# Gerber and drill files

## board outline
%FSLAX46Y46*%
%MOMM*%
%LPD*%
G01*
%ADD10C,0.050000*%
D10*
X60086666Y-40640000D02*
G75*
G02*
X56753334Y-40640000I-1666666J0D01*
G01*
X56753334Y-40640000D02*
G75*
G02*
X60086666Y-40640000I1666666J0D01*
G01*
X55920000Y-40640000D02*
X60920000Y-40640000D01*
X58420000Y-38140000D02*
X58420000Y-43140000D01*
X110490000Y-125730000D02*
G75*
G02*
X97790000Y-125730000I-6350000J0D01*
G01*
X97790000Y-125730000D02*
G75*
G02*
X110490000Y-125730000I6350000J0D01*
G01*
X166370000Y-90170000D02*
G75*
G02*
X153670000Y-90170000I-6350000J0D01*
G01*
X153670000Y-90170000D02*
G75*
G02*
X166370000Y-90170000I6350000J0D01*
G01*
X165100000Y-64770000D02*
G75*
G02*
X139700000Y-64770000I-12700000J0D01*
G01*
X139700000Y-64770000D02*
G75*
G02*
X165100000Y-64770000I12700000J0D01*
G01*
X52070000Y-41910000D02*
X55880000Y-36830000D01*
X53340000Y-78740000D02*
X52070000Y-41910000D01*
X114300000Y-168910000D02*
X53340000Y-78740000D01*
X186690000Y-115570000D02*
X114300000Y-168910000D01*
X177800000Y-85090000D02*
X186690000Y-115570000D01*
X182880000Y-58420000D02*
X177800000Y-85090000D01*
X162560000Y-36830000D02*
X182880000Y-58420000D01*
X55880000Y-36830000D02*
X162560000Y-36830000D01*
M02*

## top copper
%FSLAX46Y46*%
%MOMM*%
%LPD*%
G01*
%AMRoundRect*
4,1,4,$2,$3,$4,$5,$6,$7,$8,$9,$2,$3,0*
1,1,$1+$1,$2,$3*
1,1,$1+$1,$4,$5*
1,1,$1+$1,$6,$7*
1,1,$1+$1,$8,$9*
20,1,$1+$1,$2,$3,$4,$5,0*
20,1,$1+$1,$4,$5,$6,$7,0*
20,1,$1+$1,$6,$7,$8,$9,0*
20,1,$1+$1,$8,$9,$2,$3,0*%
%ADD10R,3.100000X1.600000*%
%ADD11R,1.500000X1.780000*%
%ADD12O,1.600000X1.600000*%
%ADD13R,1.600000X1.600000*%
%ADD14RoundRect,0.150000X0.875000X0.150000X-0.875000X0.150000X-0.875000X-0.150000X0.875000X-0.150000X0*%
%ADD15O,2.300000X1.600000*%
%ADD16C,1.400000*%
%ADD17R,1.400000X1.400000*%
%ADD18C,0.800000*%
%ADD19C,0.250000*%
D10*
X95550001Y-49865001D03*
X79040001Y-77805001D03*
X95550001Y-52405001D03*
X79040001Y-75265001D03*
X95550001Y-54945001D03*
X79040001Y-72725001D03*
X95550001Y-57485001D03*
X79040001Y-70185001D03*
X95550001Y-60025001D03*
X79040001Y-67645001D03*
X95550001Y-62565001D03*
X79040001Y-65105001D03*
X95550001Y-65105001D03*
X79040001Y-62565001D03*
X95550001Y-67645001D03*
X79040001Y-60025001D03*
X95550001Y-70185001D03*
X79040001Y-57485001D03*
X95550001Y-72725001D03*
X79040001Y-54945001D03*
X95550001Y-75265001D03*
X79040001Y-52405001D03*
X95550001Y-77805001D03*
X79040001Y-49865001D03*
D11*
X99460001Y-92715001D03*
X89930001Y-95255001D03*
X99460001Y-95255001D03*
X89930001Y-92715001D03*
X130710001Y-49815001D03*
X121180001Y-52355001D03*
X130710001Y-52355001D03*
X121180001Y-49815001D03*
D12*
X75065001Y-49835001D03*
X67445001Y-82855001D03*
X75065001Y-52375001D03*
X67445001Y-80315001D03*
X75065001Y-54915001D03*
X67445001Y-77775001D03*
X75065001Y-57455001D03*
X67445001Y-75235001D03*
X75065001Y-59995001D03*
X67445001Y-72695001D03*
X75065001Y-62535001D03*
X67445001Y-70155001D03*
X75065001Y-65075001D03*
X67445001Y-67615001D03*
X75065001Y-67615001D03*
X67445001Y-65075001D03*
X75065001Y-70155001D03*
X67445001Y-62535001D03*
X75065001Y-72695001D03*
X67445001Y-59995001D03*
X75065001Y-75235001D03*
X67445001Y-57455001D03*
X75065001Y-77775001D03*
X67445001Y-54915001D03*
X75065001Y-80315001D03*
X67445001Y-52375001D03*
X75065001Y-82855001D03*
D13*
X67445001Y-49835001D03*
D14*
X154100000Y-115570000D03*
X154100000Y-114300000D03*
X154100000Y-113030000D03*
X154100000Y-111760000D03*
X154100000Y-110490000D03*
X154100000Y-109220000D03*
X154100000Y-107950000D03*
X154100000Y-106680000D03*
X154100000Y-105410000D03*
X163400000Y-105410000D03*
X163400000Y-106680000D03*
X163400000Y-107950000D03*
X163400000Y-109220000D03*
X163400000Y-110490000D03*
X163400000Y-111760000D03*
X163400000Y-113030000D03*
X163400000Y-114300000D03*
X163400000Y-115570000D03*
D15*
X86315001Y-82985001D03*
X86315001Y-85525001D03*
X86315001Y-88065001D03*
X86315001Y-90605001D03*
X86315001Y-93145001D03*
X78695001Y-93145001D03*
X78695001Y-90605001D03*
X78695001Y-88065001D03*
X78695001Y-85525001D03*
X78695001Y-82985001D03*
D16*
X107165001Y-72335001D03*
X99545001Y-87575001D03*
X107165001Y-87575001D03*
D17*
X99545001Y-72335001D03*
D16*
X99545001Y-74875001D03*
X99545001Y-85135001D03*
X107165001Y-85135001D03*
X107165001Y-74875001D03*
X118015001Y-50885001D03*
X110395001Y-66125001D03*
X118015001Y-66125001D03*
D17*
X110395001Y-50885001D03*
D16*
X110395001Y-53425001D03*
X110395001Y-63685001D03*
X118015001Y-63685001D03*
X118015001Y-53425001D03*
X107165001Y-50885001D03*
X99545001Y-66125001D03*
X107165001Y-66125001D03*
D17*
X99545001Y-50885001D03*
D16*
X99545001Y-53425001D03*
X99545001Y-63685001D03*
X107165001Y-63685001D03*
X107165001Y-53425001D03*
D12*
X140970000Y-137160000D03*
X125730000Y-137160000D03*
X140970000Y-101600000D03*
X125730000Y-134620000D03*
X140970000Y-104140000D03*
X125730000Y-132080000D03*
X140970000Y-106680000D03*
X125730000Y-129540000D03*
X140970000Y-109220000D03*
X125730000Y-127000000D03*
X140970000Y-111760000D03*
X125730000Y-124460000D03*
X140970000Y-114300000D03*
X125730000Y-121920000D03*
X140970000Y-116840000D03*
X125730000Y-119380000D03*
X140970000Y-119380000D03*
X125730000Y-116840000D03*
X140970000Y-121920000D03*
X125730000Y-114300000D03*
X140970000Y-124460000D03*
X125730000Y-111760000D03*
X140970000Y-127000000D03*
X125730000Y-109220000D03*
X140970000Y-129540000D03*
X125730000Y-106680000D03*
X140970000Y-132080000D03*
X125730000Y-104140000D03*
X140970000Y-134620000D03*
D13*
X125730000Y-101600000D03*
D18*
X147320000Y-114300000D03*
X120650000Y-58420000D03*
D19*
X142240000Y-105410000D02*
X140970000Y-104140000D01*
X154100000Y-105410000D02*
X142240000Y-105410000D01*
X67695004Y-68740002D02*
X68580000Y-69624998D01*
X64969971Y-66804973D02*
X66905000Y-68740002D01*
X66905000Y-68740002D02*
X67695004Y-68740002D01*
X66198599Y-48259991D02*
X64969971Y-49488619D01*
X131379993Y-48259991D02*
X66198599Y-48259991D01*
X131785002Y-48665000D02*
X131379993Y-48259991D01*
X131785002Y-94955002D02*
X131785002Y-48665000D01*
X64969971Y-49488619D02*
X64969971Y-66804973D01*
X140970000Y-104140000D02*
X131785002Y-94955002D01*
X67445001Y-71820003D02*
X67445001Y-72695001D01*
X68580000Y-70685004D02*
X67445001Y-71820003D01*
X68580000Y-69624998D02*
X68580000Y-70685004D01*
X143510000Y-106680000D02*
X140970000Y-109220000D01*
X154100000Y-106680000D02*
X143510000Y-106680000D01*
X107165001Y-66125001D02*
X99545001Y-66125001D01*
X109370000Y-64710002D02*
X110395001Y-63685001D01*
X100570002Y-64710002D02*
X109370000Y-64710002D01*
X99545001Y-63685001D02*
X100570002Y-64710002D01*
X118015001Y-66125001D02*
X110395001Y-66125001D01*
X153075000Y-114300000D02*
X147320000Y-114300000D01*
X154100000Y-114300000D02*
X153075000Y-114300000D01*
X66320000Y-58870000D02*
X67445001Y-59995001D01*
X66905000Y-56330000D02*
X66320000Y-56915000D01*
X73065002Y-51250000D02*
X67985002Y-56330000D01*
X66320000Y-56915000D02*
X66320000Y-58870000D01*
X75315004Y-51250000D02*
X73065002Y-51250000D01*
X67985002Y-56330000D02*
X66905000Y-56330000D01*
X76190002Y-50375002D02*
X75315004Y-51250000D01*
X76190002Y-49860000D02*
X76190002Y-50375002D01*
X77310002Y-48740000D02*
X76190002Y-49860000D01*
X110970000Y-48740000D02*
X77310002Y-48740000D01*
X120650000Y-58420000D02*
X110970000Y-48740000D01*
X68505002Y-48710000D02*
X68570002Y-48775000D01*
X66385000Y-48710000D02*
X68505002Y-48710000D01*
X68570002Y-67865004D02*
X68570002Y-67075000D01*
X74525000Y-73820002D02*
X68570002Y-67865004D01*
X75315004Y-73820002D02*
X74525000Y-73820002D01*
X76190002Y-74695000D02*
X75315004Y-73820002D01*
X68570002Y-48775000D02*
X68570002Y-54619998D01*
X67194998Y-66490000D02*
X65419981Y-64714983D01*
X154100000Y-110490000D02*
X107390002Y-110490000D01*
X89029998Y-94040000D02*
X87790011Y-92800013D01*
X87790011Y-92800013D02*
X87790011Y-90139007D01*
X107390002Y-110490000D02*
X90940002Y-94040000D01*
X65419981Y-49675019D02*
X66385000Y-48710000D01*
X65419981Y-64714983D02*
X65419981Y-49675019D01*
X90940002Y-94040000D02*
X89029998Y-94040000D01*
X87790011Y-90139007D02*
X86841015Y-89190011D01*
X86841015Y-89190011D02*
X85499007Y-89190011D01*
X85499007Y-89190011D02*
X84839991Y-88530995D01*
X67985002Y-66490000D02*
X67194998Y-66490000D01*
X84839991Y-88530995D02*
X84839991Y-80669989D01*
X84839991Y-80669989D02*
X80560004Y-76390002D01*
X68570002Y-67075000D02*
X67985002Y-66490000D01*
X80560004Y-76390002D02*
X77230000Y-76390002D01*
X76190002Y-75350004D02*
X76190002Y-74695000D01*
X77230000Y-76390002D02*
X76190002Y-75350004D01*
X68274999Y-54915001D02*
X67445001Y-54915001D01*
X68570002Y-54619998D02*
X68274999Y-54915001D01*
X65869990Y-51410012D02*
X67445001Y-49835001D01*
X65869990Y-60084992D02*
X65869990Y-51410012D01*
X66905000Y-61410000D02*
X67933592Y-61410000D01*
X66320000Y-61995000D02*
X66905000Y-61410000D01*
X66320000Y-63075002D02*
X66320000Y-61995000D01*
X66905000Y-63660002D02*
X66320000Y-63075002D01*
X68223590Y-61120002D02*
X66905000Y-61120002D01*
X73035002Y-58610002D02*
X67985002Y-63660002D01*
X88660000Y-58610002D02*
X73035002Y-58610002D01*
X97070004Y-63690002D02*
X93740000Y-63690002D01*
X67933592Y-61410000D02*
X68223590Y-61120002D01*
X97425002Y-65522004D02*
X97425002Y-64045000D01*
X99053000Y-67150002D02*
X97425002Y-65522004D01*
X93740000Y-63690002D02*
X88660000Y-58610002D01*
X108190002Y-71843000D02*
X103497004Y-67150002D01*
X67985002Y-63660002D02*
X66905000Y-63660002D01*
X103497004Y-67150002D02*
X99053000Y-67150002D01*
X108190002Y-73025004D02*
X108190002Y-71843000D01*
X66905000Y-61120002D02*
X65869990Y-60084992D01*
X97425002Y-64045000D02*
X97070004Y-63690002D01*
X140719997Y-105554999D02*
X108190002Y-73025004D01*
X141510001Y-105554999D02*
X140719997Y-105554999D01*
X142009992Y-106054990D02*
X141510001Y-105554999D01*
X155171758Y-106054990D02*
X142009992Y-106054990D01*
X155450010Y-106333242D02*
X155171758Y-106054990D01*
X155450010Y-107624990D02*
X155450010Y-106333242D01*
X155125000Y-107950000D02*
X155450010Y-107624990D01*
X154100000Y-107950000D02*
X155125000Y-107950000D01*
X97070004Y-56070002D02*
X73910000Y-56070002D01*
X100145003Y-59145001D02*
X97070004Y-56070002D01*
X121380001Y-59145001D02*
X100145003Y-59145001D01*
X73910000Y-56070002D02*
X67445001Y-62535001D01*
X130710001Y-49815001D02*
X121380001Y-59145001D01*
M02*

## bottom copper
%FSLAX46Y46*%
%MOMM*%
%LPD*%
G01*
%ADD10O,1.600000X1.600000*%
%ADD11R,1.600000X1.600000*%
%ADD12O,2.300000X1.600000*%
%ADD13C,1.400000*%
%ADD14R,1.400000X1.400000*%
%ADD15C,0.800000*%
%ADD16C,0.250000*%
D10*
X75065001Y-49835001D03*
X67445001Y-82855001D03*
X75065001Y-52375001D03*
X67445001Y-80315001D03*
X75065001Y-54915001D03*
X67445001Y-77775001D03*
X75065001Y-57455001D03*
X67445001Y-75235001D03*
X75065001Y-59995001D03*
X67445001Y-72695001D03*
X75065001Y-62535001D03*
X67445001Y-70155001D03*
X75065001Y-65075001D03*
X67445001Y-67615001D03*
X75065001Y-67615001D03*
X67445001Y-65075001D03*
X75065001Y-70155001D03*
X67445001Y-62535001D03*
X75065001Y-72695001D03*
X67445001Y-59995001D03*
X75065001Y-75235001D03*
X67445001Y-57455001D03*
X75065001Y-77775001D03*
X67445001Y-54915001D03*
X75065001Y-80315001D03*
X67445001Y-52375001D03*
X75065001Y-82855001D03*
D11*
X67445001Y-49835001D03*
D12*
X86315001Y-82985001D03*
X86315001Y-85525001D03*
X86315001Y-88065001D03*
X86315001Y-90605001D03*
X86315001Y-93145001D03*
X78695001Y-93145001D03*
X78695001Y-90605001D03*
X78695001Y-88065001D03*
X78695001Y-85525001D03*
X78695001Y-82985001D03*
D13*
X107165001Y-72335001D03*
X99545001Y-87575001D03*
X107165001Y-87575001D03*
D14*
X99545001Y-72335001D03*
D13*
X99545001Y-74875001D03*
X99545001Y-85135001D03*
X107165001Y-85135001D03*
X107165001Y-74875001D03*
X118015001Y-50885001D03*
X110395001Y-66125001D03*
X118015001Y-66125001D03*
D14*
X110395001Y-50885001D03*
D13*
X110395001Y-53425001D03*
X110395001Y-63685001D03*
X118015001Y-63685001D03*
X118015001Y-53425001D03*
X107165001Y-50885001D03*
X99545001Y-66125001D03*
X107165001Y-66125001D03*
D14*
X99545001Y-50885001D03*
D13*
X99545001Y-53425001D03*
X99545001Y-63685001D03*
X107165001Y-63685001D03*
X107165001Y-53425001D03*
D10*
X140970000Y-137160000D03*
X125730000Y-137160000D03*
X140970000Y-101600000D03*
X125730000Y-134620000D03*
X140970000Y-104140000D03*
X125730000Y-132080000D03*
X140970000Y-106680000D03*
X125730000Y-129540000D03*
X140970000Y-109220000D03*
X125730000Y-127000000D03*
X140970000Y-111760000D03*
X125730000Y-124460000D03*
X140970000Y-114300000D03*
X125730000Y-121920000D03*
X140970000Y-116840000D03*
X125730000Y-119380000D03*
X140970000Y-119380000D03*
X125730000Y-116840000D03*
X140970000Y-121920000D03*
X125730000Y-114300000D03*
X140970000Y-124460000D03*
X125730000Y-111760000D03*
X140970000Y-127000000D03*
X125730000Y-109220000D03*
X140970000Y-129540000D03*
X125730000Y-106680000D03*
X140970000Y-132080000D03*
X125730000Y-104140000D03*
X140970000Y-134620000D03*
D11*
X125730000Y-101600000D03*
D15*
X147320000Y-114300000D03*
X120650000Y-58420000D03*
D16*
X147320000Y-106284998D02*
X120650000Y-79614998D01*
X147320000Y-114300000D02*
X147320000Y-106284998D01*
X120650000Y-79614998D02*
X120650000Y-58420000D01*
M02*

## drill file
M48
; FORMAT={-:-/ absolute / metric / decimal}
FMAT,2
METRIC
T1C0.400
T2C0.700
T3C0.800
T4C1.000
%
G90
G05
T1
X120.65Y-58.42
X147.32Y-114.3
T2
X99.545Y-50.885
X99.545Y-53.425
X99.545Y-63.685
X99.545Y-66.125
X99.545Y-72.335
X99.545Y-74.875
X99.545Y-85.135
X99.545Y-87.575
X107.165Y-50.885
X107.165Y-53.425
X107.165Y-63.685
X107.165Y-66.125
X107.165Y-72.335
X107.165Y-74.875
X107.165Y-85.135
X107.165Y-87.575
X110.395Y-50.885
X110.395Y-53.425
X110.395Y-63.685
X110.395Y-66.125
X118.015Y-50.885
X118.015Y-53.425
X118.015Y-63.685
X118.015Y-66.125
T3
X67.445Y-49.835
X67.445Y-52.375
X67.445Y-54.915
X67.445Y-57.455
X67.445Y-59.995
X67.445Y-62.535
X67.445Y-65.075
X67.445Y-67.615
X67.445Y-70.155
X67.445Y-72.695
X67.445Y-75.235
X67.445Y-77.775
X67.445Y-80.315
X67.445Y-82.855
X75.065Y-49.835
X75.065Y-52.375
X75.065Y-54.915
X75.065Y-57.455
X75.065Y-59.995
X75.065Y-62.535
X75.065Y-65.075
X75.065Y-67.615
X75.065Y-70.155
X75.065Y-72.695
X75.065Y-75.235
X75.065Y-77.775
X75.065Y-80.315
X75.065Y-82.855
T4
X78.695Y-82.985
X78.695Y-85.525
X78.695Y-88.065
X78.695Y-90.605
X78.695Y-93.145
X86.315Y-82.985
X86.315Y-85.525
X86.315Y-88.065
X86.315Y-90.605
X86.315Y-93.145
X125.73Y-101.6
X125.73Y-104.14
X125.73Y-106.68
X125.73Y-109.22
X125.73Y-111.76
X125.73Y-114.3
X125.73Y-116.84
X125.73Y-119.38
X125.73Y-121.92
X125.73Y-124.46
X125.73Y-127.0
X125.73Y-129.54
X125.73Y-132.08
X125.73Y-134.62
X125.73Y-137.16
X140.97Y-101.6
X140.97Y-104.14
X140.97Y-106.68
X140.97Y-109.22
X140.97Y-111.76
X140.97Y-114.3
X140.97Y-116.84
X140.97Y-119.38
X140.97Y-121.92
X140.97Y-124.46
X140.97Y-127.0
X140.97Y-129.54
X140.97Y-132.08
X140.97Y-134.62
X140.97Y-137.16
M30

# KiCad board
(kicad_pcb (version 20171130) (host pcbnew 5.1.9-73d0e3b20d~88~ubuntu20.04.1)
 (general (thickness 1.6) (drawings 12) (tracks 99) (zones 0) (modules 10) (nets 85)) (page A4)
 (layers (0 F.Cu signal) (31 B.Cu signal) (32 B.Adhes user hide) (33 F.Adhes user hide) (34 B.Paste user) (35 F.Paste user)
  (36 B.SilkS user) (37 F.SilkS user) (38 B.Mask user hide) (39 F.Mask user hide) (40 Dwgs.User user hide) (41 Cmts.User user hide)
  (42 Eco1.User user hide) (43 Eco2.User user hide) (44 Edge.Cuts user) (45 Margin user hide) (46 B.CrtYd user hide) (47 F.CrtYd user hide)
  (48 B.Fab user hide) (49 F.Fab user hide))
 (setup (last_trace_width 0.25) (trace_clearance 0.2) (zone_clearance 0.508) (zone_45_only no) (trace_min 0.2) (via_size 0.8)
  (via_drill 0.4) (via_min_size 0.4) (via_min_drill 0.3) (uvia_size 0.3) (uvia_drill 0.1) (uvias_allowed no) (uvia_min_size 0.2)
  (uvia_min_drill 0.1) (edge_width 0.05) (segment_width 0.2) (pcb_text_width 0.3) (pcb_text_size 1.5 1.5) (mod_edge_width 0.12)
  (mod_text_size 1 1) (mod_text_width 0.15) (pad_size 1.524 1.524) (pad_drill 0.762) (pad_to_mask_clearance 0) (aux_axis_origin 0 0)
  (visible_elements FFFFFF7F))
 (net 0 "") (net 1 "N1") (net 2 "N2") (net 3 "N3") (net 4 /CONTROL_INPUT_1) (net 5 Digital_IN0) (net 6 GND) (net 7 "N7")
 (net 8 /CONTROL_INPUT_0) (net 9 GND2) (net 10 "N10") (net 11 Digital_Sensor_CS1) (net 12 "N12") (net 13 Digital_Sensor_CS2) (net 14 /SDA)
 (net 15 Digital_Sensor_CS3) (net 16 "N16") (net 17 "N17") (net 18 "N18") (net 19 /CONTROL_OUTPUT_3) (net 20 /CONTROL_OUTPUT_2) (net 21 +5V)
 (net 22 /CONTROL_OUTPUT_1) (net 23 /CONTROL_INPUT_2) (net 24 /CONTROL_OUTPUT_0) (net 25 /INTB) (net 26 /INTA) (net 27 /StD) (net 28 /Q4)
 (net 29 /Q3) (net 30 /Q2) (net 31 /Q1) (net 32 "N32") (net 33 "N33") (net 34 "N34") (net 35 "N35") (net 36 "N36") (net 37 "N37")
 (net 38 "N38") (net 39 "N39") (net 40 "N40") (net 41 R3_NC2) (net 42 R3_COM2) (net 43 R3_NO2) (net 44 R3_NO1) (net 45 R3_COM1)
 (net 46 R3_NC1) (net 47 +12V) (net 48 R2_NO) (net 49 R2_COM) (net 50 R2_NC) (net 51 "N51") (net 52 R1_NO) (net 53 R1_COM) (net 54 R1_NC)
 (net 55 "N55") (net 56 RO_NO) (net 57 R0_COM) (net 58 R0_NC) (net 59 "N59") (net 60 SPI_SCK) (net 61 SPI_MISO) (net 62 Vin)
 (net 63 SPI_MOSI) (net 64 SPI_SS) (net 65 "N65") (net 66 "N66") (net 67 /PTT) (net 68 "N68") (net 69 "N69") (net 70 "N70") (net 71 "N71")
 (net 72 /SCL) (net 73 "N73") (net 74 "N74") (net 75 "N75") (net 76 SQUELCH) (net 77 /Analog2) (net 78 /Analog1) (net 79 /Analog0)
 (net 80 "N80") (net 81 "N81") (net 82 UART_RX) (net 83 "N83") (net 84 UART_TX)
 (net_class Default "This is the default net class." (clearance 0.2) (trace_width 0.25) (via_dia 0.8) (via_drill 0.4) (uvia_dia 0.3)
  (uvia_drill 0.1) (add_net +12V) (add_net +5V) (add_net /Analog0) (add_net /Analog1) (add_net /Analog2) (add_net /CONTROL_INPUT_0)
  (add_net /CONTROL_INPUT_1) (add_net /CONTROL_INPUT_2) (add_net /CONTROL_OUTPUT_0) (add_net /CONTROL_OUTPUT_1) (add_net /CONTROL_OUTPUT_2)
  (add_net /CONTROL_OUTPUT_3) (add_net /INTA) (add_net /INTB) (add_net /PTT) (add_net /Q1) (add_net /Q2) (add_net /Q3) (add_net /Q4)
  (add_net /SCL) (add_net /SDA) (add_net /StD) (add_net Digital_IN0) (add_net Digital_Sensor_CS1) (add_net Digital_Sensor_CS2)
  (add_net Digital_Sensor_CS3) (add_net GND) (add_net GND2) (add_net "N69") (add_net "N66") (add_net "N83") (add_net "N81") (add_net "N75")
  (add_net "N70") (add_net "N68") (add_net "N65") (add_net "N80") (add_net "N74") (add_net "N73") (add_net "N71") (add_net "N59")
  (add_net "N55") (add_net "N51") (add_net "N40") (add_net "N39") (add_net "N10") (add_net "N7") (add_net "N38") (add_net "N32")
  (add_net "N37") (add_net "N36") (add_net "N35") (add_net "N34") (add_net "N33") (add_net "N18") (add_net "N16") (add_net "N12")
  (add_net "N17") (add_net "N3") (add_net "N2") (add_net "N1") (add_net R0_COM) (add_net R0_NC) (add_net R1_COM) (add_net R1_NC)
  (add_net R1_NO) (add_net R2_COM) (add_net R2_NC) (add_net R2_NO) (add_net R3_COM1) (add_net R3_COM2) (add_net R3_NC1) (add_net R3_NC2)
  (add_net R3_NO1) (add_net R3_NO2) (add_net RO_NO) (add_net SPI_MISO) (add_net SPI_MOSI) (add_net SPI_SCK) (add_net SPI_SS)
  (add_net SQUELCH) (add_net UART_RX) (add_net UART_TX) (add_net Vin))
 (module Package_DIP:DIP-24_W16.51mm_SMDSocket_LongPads (layer F.Cu) (at 87.295001 63.835001)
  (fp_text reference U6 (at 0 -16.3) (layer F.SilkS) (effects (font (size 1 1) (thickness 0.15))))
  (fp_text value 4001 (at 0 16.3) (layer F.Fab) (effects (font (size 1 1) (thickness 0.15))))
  (pad 24 smd rect (at 8.255 -13.97) (size 3.1 1.6) (layers F.Cu F.Paste F.Mask))
  (pad 12 smd rect (at -8.255 13.97) (size 3.1 1.6) (layers F.Cu F.Paste F.Mask))
  (pad 23 smd rect (at 8.255 -11.43) (size 3.1 1.6) (layers F.Cu F.Paste F.Mask))
  (pad 11 smd rect (at -8.255 11.43) (size 3.1 1.6) (layers F.Cu F.Paste F.Mask))
  (pad 22 smd rect (at 8.255 -8.89) (size 3.1 1.6) (layers F.Cu F.Paste F.Mask))
  (pad 10 smd rect (at -8.255 8.89) (size 3.1 1.6) (layers F.Cu F.Paste F.Mask))
  (pad 21 smd rect (at 8.255 -6.35) (size 3.1 1.6) (layers F.Cu F.Paste F.Mask))
  (pad 9 smd rect (at -8.255 6.35) (size 3.1 1.6) (layers F.Cu F.Paste F.Mask))
  (pad 20 smd rect (at 8.255 -3.81) (size 3.1 1.6) (layers F.Cu F.Paste F.Mask))
  (pad 8 smd rect (at -8.255 3.81) (size 3.1 1.6) (layers F.Cu F.Paste F.Mask))
  (pad 19 smd rect (at 8.255 -1.27) (size 3.1 1.6) (layers F.Cu F.Paste F.Mask))
  (pad 7 smd rect (at -8.255 1.27) (size 3.1 1.6) (layers F.Cu F.Paste F.Mask))
  (pad 18 smd rect (at 8.255 1.27) (size 3.1 1.6) (layers F.Cu F.Paste F.Mask))
  (pad 6 smd rect (at -8.255 -1.27) (size 3.1 1.6) (layers F.Cu F.Paste F.Mask))
  (pad 17 smd rect (at 8.255 3.81) (size 3.1 1.6) (layers F.Cu F.Paste F.Mask))
  (pad 5 smd rect (at -8.255 -3.81) (size 3.1 1.6) (layers F.Cu F.Paste F.Mask))
  (pad 16 smd rect (at 8.255 6.35) (size 3.1 1.6) (layers F.Cu F.Paste F.Mask))
  (pad 4 smd rect (at -8.255 -6.35) (size 3.1 1.6) (layers F.Cu F.Paste F.Mask))
  (pad 15 smd rect (at 8.255 8.89) (size 3.1 1.6) (layers F.Cu F.Paste F.Mask))
  (pad 3 smd rect (at -8.255 -8.89) (size 3.1 1.6) (layers F.Cu F.Paste F.Mask) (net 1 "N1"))
  (pad 14 smd rect (at 8.255 11.43) (size 3.1 1.6) (layers F.Cu F.Paste F.Mask))
  (pad 2 smd rect (at -8.255 -11.43) (size 3.1 1.6) (layers F.Cu F.Paste F.Mask) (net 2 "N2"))
  (pad 13 smd rect (at 8.255 13.97) (size 3.1 1.6) (layers F.Cu F.Paste F.Mask))
  (pad 1 smd rect (at -8.255 -13.97) (size 3.1 1.6) (layers F.Cu F.Paste F.Mask) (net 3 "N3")))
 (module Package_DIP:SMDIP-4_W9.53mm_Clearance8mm (layer F.Cu) (at 94.695001 93.985001)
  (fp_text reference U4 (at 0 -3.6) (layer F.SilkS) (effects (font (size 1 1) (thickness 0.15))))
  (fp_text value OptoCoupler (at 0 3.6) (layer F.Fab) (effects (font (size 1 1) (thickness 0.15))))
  (pad 4 smd rect (at 4.765 -1.27) (size 1.5 1.78) (layers F.Cu F.Paste F.Mask) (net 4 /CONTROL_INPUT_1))
  (pad 2 smd rect (at -4.765 1.27) (size 1.5 1.78) (layers F.Cu F.Paste F.Mask) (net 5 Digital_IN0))
  (pad 3 smd rect (at 4.765 1.27) (size 1.5 1.78) (layers F.Cu F.Paste F.Mask) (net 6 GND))
  (pad 1 smd rect (at -4.765 -1.27) (size 1.5 1.78) (layers F.Cu F.Paste F.Mask) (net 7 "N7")))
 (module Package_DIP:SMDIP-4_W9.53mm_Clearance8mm (layer F.Cu) (at 125.945001 51.085001)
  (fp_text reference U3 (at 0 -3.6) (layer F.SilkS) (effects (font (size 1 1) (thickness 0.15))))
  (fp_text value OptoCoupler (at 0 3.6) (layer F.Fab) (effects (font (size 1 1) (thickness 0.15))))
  (pad 4 smd rect (at 4.765 -1.27) (size 1.5 1.78) (layers F.Cu F.Paste F.Mask) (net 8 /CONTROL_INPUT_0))
  (pad 2 smd rect (at -4.765 1.27) (size 1.5 1.78) (layers F.Cu F.Paste F.Mask) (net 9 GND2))
  (pad 3 smd rect (at 4.765 1.27) (size 1.5 1.78) (layers F.Cu F.Paste F.Mask) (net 6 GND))
  (pad 1 smd rect (at -4.765 -1.27) (size 1.5 1.78) (layers F.Cu F.Paste F.Mask) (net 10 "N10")))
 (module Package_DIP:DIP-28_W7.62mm (layer F.Cu) (at 67.445001 49.835001)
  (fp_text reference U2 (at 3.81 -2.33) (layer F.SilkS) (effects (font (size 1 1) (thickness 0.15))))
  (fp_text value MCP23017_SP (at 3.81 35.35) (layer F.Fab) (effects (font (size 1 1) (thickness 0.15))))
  (pad 28 thru_hole oval (at 7.62 0) (size 1.6 1.6) (drill 0.8) (layers *.Cu *.Mask) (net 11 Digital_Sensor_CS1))
  (pad 14 thru_hole oval (at 0 33.02) (size 1.6 1.6) (drill 0.8) (layers *.Cu *.Mask) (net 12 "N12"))
  (pad 27 thru_hole oval (at 7.62 2.54) (size 1.6 1.6) (drill 0.8) (layers *.Cu *.Mask) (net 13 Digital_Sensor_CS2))
  (pad 13 thru_hole oval (at 0 30.48) (size 1.6 1.6) (drill 0.8) (layers *.Cu *.Mask) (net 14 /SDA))
  (pad 26 thru_hole oval (at 7.62 5.08) (size 1.6 1.6) (drill 0.8) (layers *.Cu *.Mask) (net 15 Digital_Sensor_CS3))
  (pad 12 thru_hole oval (at 0 27.94) (size 1.6 1.6) (drill 0.8) (layers *.Cu *.Mask) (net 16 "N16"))
  (pad 25 thru_hole oval (at 7.62 7.62) (size 1.6 1.6) (drill 0.8) (layers *.Cu *.Mask) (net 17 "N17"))
  (pad 11 thru_hole oval (at 0 25.4) (size 1.6 1.6) (drill 0.8) (layers *.Cu *.Mask) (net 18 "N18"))
  (pad 24 thru_hole oval (at 7.62 10.16) (size 1.6 1.6) (drill 0.8) (layers *.Cu *.Mask) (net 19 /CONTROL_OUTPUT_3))
  (pad 10 thru_hole oval (at 0 22.86) (size 1.6 1.6) (drill 0.8) (layers *.Cu *.Mask) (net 6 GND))
  (pad 23 thru_hole oval (at 7.62 12.7) (size 1.6 1.6) (drill 0.8) (layers *.Cu *.Mask) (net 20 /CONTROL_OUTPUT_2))
  (pad 9 thru_hole oval (at 0 20.32) (size 1.6 1.6) (drill 0.8) (layers *.Cu *.Mask) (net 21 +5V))
  (pad 22 thru_hole oval (at 7.62 15.24) (size 1.6 1.6) (drill 0.8) (layers *.Cu *.Mask) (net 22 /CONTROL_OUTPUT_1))
  (pad 8 thru_hole oval (at 0 17.78) (size 1.6 1.6) (drill 0.8) (layers *.Cu *.Mask) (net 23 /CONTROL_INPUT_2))
  (pad 21 thru_hole oval (at 7.62 17.78) (size 1.6 1.6) (drill 0.8) (layers *.Cu *.Mask) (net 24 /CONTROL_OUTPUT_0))
  (pad 7 thru_hole oval (at 0 15.24) (size 1.6 1.6) (drill 0.8) (layers *.Cu *.Mask) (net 4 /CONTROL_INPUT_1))
  (pad 20 thru_hole oval (at 7.62 20.32) (size 1.6 1.6) (drill 0.8) (layers *.Cu *.Mask) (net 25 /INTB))
  (pad 6 thru_hole oval (at 0 12.7) (size 1.6 1.6) (drill 0.8) (layers *.Cu *.Mask) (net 8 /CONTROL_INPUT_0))
  (pad 19 thru_hole oval (at 7.62 22.86) (size 1.6 1.6) (drill 0.8) (layers *.Cu *.Mask) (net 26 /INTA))
  (pad 5 thru_hole oval (at 0 10.16) (size 1.6 1.6) (drill 0.8) (layers *.Cu *.Mask) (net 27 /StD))
  (pad 18 thru_hole oval (at 7.62 25.4) (size 1.6 1.6) (drill 0.8) (layers *.Cu *.Mask) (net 21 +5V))
  (pad 4 thru_hole oval (at 0 7.62) (size 1.6 1.6) (drill 0.8) (layers *.Cu *.Mask) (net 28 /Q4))
  (pad 17 thru_hole oval (at 7.62 27.94) (size 1.6 1.6) (drill 0.8) (layers *.Cu *.Mask) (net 6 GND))
  (pad 3 thru_hole oval (at 0 5.08) (size 1.6 1.6) (drill 0.8) (layers *.Cu *.Mask) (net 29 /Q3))
  (pad 16 thru_hole oval (at 7.62 30.48) (size 1.6 1.6) (drill 0.8) (layers *.Cu *.Mask) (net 6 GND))
  (pad 2 thru_hole oval (at 0 2.54) (size 1.6 1.6) (drill 0.8) (layers *.Cu *.Mask) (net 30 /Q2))
  (pad 15 thru_hole oval (at 7.62 33.02) (size 1.6 1.6) (drill 0.8) (layers *.Cu *.Mask) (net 6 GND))
  (pad 1 thru_hole rect (at 0 0) (size 1.6 1.6) (drill 0.8) (layers *.Cu *.Mask) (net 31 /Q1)))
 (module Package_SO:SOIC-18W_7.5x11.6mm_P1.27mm (layer F.Cu) (at 158.75 110.49 180)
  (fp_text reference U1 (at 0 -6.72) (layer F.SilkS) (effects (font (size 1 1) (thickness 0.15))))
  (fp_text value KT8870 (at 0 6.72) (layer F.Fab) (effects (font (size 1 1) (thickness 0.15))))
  (pad 18 smd roundrect (at 4.65 -5.08 180) (size 2.05 0.6) (layers F.Cu F.Paste F.Mask) (roundrect_rratio 0.25) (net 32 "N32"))
  (pad 17 smd roundrect (at 4.65 -3.81 180) (size 2.05 0.6) (layers F.Cu F.Paste F.Mask) (roundrect_rratio 0.25) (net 27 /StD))
  (pad 16 smd roundrect (at 4.65 -2.54 180) (size 2.05 0.6) (layers F.Cu F.Paste F.Mask) (roundrect_rratio 0.25))
  (pad 15 smd roundrect (at 4.65 -1.27 180) (size 2.05 0.6) (layers F.Cu F.Paste F.Mask) (roundrect_rratio 0.25) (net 28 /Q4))
  (pad 14 smd roundrect (at 4.65 0 180) (size 2.05 0.6) (layers F.Cu F.Paste F.Mask) (roundrect_rratio 0.25) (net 29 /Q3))
  (pad 13 smd roundrect (at 4.65 1.27 180) (size 2.05 0.6) (layers F.Cu F.Paste F.Mask) (roundrect_rratio 0.25) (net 30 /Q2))
  (pad 12 smd roundrect (at 4.65 2.54 180) (size 2.05 0.6) (layers F.Cu F.Paste F.Mask) (roundrect_rratio 0.25) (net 31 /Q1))
  (pad 11 smd roundrect (at 4.65 3.81 180) (size 2.05 0.6) (layers F.Cu F.Paste F.Mask) (roundrect_rratio 0.25) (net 21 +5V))
  (pad 10 smd roundrect (at 4.65 5.08 180) (size 2.05 0.6) (layers F.Cu F.Paste F.Mask) (roundrect_rratio 0.25) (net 6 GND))
  (pad 9 smd roundrect (at -4.65 5.08 180) (size 2.05 0.6) (layers F.Cu F.Paste F.Mask) (roundrect_rratio 0.25) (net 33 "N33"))
  (pad 8 smd roundrect (at -4.65 3.81 180) (size 2.05 0.6) (layers F.Cu F.Paste F.Mask) (roundrect_rratio 0.25) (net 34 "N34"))
  (pad 7 smd roundrect (at -4.65 2.54 180) (size 2.05 0.6) (layers F.Cu F.Paste F.Mask) (roundrect_rratio 0.25))
  (pad 6 smd roundrect (at -4.65 1.27 180) (size 2.05 0.6) (layers F.Cu F.Paste F.Mask) (roundrect_rratio 0.25) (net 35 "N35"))
  (pad 5 smd roundrect (at -4.65 0 180) (size 2.05 0.6) (layers F.Cu F.Paste F.Mask) (roundrect_rratio 0.25) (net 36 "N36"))
  (pad 4 smd roundrect (at -4.65 -1.27 180) (size 2.05 0.6) (layers F.Cu F.Paste F.Mask) (roundrect_rratio 0.25) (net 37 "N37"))
  (pad 3 smd roundrect (at -4.65 -2.54 180) (size 2.05 0.6) (layers F.Cu F.Paste F.Mask) (roundrect_rratio 0.25) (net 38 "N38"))
  (pad 2 smd roundrect (at -4.65 -3.81 180) (size 2.05 0.6) (layers F.Cu F.Paste F.Mask) (roundrect_rratio 0.25) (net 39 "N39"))
  (pad 1 smd roundrect (at -4.65 -5.08 180) (size 2.05 0.6) (layers F.Cu F.Paste F.Mask) (roundrect_rratio 0.25) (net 37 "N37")))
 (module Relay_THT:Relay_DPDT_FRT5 (layer F.Cu) (at 78.695001 82.985001)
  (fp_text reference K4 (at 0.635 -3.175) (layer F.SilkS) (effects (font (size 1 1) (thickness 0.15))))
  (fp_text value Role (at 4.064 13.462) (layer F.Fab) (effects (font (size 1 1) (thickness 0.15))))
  (pad 10 thru_hole oval (at 7.62 0) (size 2.3 1.6) (drill 1) (layers *.Cu *.Mask) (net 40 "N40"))
  (pad 9 thru_hole oval (at 7.62 2.54) (size 2.3 1.6) (drill 1) (layers *.Cu *.Mask) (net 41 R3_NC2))
  (pad 8 thru_hole oval (at 7.62 5.08) (size 2.3 1.6) (drill 1) (layers *.Cu *.Mask) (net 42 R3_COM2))
  (pad 7 thru_hole oval (at 7.62 7.62) (size 2.3 1.6) (drill 1) (layers *.Cu *.Mask) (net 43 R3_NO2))
  (pad 6 thru_hole oval (at 7.62 10.16) (size 2.3 1.6) (drill 1) (layers *.Cu *.Mask))
  (pad 5 thru_hole oval (at 0 10.16) (size 2.3 1.6) (drill 1) (layers *.Cu *.Mask))
  (pad 4 thru_hole oval (at 0 7.62) (size 2.3 1.6) (drill 1) (layers *.Cu *.Mask) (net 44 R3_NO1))
  (pad 3 thru_hole oval (at 0 5.08) (size 2.3 1.6) (drill 1) (layers *.Cu *.Mask) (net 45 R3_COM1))
  (pad 2 thru_hole oval (at 0 2.54) (size 2.3 1.6) (drill 1) (layers *.Cu *.Mask) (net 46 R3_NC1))
  (pad 1 thru_hole oval (at 0 0) (size 2.3 1.6) (drill 1) (layers *.Cu *.Mask) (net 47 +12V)))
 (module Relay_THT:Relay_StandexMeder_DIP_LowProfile (layer F.Cu) (at 99.545001 72.335001)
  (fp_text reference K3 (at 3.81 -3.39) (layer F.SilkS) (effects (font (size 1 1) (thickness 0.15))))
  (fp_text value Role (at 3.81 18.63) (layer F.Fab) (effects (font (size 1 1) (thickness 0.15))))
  (pad 14 thru_hole circle (at 7.62 0) (size 1.4 1.4) (drill 0.7) (layers *.Cu *.Mask) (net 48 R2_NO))
  (pad 7 thru_hole circle (at 0 15.24) (size 1.4 1.4) (drill 0.7) (layers *.Cu *.Mask) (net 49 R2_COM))
  (pad 8 thru_hole circle (at 7.62 15.24) (size 1.4 1.4) (drill 0.7) (layers *.Cu *.Mask) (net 49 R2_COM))
  (pad 1 thru_hole rect (at 0 0) (size 1.4 1.4) (drill 0.7) (layers *.Cu *.Mask) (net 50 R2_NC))
  (pad 2 thru_hole circle (at 0 2.54) (size 1.4 1.4) (drill 0.7) (layers *.Cu *.Mask) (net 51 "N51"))
  (pad 6 thru_hole circle (at 0 12.8) (size 1.4 1.4) (drill 0.7) (layers *.Cu *.Mask) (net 47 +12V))
  (pad 9 thru_hole circle (at 7.62 12.8) (size 1.4 1.4) (drill 0.7) (layers *.Cu *.Mask))
  (pad 13 thru_hole circle (at 7.62 2.54) (size 1.4 1.4) (drill 0.7) (layers *.Cu *.Mask)))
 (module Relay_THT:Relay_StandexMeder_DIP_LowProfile (layer F.Cu) (at 110.395001 50.885001)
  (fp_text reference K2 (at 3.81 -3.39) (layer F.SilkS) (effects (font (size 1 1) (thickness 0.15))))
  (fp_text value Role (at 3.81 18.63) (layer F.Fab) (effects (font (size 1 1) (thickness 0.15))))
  (pad 14 thru_hole circle (at 7.62 0) (size 1.4 1.4) (drill 0.7) (layers *.Cu *.Mask) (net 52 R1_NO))
  (pad 7 thru_hole circle (at 0 15.24) (size 1.4 1.4) (drill 0.7) (layers *.Cu *.Mask) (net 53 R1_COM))
  (pad 8 thru_hole circle (at 7.62 15.24) (size 1.4 1.4) (drill 0.7) (layers *.Cu *.Mask) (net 53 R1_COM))
  (pad 1 thru_hole rect (at 0 0) (size 1.4 1.4) (drill 0.7) (layers *.Cu *.Mask) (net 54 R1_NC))
  (pad 2 thru_hole circle (at 0 2.54) (size 1.4 1.4) (drill 0.7) (layers *.Cu *.Mask) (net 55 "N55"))
  (pad 6 thru_hole circle (at 0 12.8) (size 1.4 1.4) (drill 0.7) (layers *.Cu *.Mask) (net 47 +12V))
  (pad 9 thru_hole circle (at 7.62 12.8) (size 1.4 1.4) (drill 0.7) (layers *.Cu *.Mask))
  (pad 13 thru_hole circle (at 7.62 2.54) (size 1.4 1.4) (drill 0.7) (layers *.Cu *.Mask)))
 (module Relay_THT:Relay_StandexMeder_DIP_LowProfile (layer F.Cu) (at 99.545001 50.885001)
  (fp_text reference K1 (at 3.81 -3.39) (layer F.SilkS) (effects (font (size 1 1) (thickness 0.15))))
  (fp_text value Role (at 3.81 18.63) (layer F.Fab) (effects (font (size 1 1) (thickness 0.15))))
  (pad 14 thru_hole circle (at 7.62 0) (size 1.4 1.4) (drill 0.7) (layers *.Cu *.Mask) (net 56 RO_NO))
  (pad 7 thru_hole circle (at 0 15.24) (size 1.4 1.4) (drill 0.7) (layers *.Cu *.Mask) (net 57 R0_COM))
  (pad 8 thru_hole circle (at 7.62 15.24) (size 1.4 1.4) (drill 0.7) (layers *.Cu *.Mask) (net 57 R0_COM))
  (pad 1 thru_hole rect (at 0 0) (size 1.4 1.4) (drill 0.7) (layers *.Cu *.Mask) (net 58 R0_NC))
  (pad 2 thru_hole circle (at 0 2.54) (size 1.4 1.4) (drill 0.7) (layers *.Cu *.Mask) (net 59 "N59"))
  (pad 6 thru_hole circle (at 0 12.8) (size 1.4 1.4) (drill 0.7) (layers *.Cu *.Mask) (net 47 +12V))
  (pad 9 thru_hole circle (at 7.62 12.8) (size 1.4 1.4) (drill 0.7) (layers *.Cu *.Mask))
  (pad 13 thru_hole circle (at 7.62 2.54) (size 1.4 1.4) (drill 0.7) (layers *.Cu *.Mask)))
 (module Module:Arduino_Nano (layer F.Cu) (at 125.73 101.6)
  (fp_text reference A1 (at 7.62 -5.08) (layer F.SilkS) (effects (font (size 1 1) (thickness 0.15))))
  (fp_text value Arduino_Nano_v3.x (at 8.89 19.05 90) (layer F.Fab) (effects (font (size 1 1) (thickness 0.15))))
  (pad 16 thru_hole oval (at 15.24 35.56) (size 1.6 1.6) (drill 1) (layers *.Cu *.Mask) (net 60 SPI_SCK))
  (pad 15 thru_hole oval (at 0 35.56) (size 1.6 1.6) (drill 1) (layers *.Cu *.Mask) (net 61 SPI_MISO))
  (pad 30 thru_hole oval (at 15.24 0) (size 1.6 1.6) (drill 1) (layers *.Cu *.Mask) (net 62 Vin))
  (pad 14 thru_hole oval (at 0 33.02) (size 1.6 1.6) (drill 1) (layers *.Cu *.Mask) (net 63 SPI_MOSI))
  (pad 29 thru_hole oval (at 15.24 2.54) (size 1.6 1.6) (drill 1) (layers *.Cu *.Mask) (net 6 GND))
  (pad 13 thru_hole oval (at 0 30.48) (size 1.6 1.6) (drill 1) (layers *.Cu *.Mask) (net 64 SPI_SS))
  (pad 28 thru_hole oval (at 15.24 5.08) (size 1.6 1.6) (drill 1) (layers *.Cu *.Mask) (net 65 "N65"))
  (pad 12 thru_hole oval (at 0 27.94) (size 1.6 1.6) (drill 1) (layers *.Cu *.Mask) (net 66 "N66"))
  (pad 27 thru_hole oval (at 15.24 7.62) (size 1.6 1.6) (drill 1) (layers *.Cu *.Mask) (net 21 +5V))
  (pad 11 thru_hole oval (at 0 25.4) (size 1.6 1.6) (drill 1) (layers *.Cu *.Mask) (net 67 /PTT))
  (pad 26 thru_hole oval (at 15.24 10.16) (size 1.6 1.6) (drill 1) (layers *.Cu *.Mask) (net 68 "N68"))
  (pad 10 thru_hole oval (at 0 22.86) (size 1.6 1.6) (drill 1) (layers *.Cu *.Mask) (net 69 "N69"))
  (pad 25 thru_hole oval (at 15.24 12.7) (size 1.6 1.6) (drill 1) (layers *.Cu *.Mask) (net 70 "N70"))
  (pad 9 thru_hole oval (at 0 20.32) (size 1.6 1.6) (drill 1) (layers *.Cu *.Mask) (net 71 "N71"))
  (pad 24 thru_hole oval (at 15.24 15.24) (size 1.6 1.6) (drill 1) (layers *.Cu *.Mask) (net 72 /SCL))
  (pad 8 thru_hole oval (at 0 17.78) (size 1.6 1.6) (drill 1) (layers *.Cu *.Mask) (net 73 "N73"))
  (pad 23 thru_hole oval (at 15.24 17.78) (size 1.6 1.6) (drill 1) (layers *.Cu *.Mask) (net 14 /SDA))
  (pad 7 thru_hole oval (at 0 15.24) (size 1.6 1.6) (drill 1) (layers *.Cu *.Mask) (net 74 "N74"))
  (pad 22 thru_hole oval (at 15.24 20.32) (size 1.6 1.6) (drill 1) (layers *.Cu *.Mask) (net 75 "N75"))
  (pad 6 thru_hole oval (at 0 12.7) (size 1.6 1.6) (drill 1) (layers *.Cu *.Mask) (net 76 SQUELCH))
  (pad 21 thru_hole oval (at 15.24 22.86) (size 1.6 1.6) (drill 1) (layers *.Cu *.Mask) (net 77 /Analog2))
  (pad 5 thru_hole oval (at 0 10.16) (size 1.6 1.6) (drill 1) (layers *.Cu *.Mask) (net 26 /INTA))
  (pad 20 thru_hole oval (at 15.24 25.4) (size 1.6 1.6) (drill 1) (layers *.Cu *.Mask) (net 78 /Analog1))
  (pad 4 thru_hole oval (at 0 7.62) (size 1.6 1.6) (drill 1) (layers *.Cu *.Mask) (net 6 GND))
  (pad 19 thru_hole oval (at 15.24 27.94) (size 1.6 1.6) (drill 1) (layers *.Cu *.Mask) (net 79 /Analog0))
  (pad 3 thru_hole oval (at 0 5.08) (size 1.6 1.6) (drill 1) (layers *.Cu *.Mask) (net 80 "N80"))
  (pad 18 thru_hole oval (at 15.24 30.48) (size 1.6 1.6) (drill 1) (layers *.Cu *.Mask) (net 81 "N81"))
  (pad 2 thru_hole oval (at 0 2.54) (size 1.6 1.6) (drill 1) (layers *.Cu *.Mask) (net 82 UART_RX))
  (pad 17 thru_hole oval (at 15.24 33.02) (size 1.6 1.6) (drill 1) (layers *.Cu *.Mask) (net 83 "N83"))
  (pad 1 thru_hole rect (at 0 0) (size 1.6 1.6) (drill 1) (layers *.Cu *.Mask) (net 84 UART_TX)))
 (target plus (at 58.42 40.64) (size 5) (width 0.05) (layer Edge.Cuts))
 (gr_circle (center 104.14 125.73) (end 107.95 130.81) (layer Edge.Cuts) (width 0.05))
 (gr_circle (center 160.02 90.17) (end 163.83 95.25) (layer Edge.Cuts) (width 0.05))
 (gr_circle (center 152.4 64.77) (end 160.02 74.93) (layer Edge.Cuts) (width 0.05))
 (gr_line (start 52.07 41.91) (end 55.88 36.83) (layer Edge.Cuts) (width 0.05))
 (gr_line (start 53.34 78.74) (end 52.07 41.91) (layer Edge.Cuts) (width 0.05))
 (gr_line (start 114.3 168.91) (end 53.34 78.74) (layer Edge.Cuts) (width 0.05))
 (gr_line (start 186.69 115.57) (end 114.3 168.91) (layer Edge.Cuts) (width 0.05))
 (gr_line (start 177.8 85.09) (end 186.69 115.57) (layer Edge.Cuts) (width 0.05))
 (gr_line (start 182.88 58.42) (end 177.8 85.09) (layer Edge.Cuts) (width 0.05))
 (gr_line (start 162.56 36.83) (end 182.88 58.42) (layer Edge.Cuts) (width 0.05))
 (gr_line (start 55.88 36.83) (end 162.56 36.83) (layer Edge.Cuts) (width 0.05))
 (segment (start 142.24 105.41) (end 140.97 104.14) (width 0.25) (layer F.Cu) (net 6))
 (segment (start 154.1 105.41) (end 142.24 105.41) (width 0.25) (layer F.Cu) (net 6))
 (segment (start 67.695004 68.740002) (end 68.58 69.624998) (width 0.25) (layer F.Cu) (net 6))
 (segment (start 64.969971 66.804973) (end 66.905 68.740002) (width 0.25) (layer F.Cu) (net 6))
 (segment (start 66.905 68.740002) (end 67.695004 68.740002) (width 0.25) (layer F.Cu) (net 6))
 (segment (start 66.198599 48.259991) (end 64.969971 49.488619) (width 0.25) (layer F.Cu) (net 6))
 (segment (start 131.379993 48.259991) (end 66.198599 48.259991) (width 0.25) (layer F.Cu) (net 6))
 (segment (start 131.785002 48.665) (end 131.379993 48.259991) (width 0.25) (layer F.Cu) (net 6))
 (segment (start 131.785002 94.955002) (end 131.785002 48.665) (width 0.25) (layer F.Cu) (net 6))
 (segment (start 64.969971 49.488619) (end 64.969971 66.804973) (width 0.25) (layer F.Cu) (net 6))
 (segment (start 140.97 104.14) (end 131.785002 94.955002) (width 0.25) (layer F.Cu) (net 6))
 (segment (start 67.445001 71.820003) (end 67.445001 72.695001) (width 0.25) (layer F.Cu) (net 6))
 (segment (start 68.58 70.685004) (end 67.445001 71.820003) (width 0.25) (layer F.Cu) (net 6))
 (segment (start 68.58 69.624998) (end 68.58 70.685004) (width 0.25) (layer F.Cu) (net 6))
 (segment (start 143.51 106.68) (end 140.97 109.22) (width 0.25) (layer F.Cu) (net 21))
 (segment (start 154.1 106.68) (end 143.51 106.68) (width 0.25) (layer F.Cu) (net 21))
 (segment (start 107.165001 66.125001) (end 99.545001 66.125001) (width 0.25) (layer F.Cu) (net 57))
 (segment (start 109.37 64.710002) (end 110.395001 63.685001) (width 0.25) (layer F.Cu) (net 47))
 (segment (start 100.570002 64.710002) (end 109.37 64.710002) (width 0.25) (layer F.Cu) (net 47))
 (segment (start 99.545001 63.685001) (end 100.570002 64.710002) (width 0.25) (layer F.Cu) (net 47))
 (segment (start 118.015001 66.125001) (end 110.395001 66.125001) (width 0.25) (layer F.Cu) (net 53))
 (via (at 147.32 114.3) (size 0.8) (drill 0.4) (layers F.Cu B.Cu) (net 27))
 (segment (start 153.075 114.3) (end 147.32 114.3) (width 0.25) (layer F.Cu) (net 27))
 (segment (start 154.1 114.3) (end 153.075 114.3) (width 0.25) (layer F.Cu) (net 27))
 (segment (start 147.32 106.284998) (end 120.65 79.614998) (width 0.25) (layer B.Cu) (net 27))
 (segment (start 147.32 114.3) (end 147.32 106.284998) (width 0.25) (layer B.Cu) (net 27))
 (segment (start 120.65 79.614998) (end 120.65 58.42) (width 0.25) (layer B.Cu) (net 27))
 (via (at 120.65 58.42) (size 0.8) (drill 0.4) (layers F.Cu B.Cu) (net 27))
 (segment (start 66.32 58.87) (end 67.445001 59.995001) (width 0.25) (layer F.Cu) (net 27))
 (segment (start 66.905 56.33) (end 66.32 56.915) (width 0.25) (layer F.Cu) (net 27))
 (segment (start 73.065002 51.25) (end 67.985002 56.33) (width 0.25) (layer F.Cu) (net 27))
 (segment (start 66.32 56.915) (end 66.32 58.87) (width 0.25) (layer F.Cu) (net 27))
 (segment (start 75.315004 51.25) (end 73.065002 51.25) (width 0.25) (layer F.Cu) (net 27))
 (segment (start 67.985002 56.33) (end 66.905 56.33) (width 0.25) (layer F.Cu) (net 27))
 (segment (start 76.190002 50.375002) (end 75.315004 51.25) (width 0.25) (layer F.Cu) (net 27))
 (segment (start 76.190002 49.86) (end 76.190002 50.375002) (width 0.25) (layer F.Cu) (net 27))
 (segment (start 77.310002 48.74) (end 76.190002 49.86) (width 0.25) (layer F.Cu) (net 27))
 (segment (start 110.97 48.74) (end 77.310002 48.74) (width 0.25) (layer F.Cu) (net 27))
 (segment (start 120.65 58.42) (end 110.97 48.74) (width 0.25) (layer F.Cu) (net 27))
 (segment (start 68.505002 48.71) (end 68.570002 48.775) (width 0.25) (layer F.Cu) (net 29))
 (segment (start 66.385 48.71) (end 68.505002 48.71) (width 0.25) (layer F.Cu) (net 29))
 (segment (start 68.570002 67.865004) (end 68.570002 67.075) (width 0.25) (layer F.Cu) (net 29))
 (segment (start 74.525 73.820002) (end 68.570002 67.865004) (width 0.25) (layer F.Cu) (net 29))
 (segment (start 75.315004 73.820002) (end 74.525 73.820002) (width 0.25) (layer F.Cu) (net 29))
 (segment (start 76.190002 74.695) (end 75.315004 73.820002) (width 0.25) (layer F.Cu) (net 29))
 (segment (start 68.570002 48.775) (end 68.570002 54.619998) (width 0.25) (layer F.Cu) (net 29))
 (segment (start 67.194998 66.49) (end 65.419981 64.714983) (width 0.25) (layer F.Cu) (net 29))
 (segment (start 154.1 110.49) (end 107.390002 110.49) (width 0.25) (layer F.Cu) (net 29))
 (segment (start 89.029998 94.04) (end 87.790011 92.800013) (width 0.25) (layer F.Cu) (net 29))
 (segment (start 87.790011 92.800013) (end 87.790011 90.139007) (width 0.25) (layer F.Cu) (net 29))
 (segment (start 107.390002 110.49) (end 90.940002 94.04) (width 0.25) (layer F.Cu) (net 29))
 (segment (start 65.419981 49.675019) (end 66.385 48.71) (width 0.25) (layer F.Cu) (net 29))
 (segment (start 65.419981 64.714983) (end 65.419981 49.675019) (width 0.25) (layer F.Cu) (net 29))
 (segment (start 90.940002 94.04) (end 89.029998 94.04) (width 0.25) (layer F.Cu) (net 29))
 (segment (start 87.790011 90.139007) (end 86.841015 89.190011) (width 0.25) (layer F.Cu) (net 29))
 (segment (start 86.841015 89.190011) (end 85.499007 89.190011) (width 0.25) (layer F.Cu) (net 29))
 (segment (start 85.499007 89.190011) (end 84.839991 88.530995) (width 0.25) (layer F.Cu) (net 29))
 (segment (start 67.985002 66.49) (end 67.194998 66.49) (width 0.25) (layer F.Cu) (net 29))
 (segment (start 84.839991 88.530995) (end 84.839991 80.669989) (width 0.25) (layer F.Cu) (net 29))
 (segment (start 84.839991 80.669989) (end 80.560004 76.390002) (width 0.25) (layer F.Cu) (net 29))
 (segment (start 68.570002 67.075) (end 67.985002 66.49) (width 0.25) (layer F.Cu) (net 29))
 (segment (start 80.560004 76.390002) (end 77.23 76.390002) (width 0.25) (layer F.Cu) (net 29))
 (segment (start 76.190002 75.350004) (end 76.190002 74.695) (width 0.25) (layer F.Cu) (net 29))
 (segment (start 77.23 76.390002) (end 76.190002 75.350004) (width 0.25) (layer F.Cu) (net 29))
 (segment (start 68.274999 54.915001) (end 67.445001 54.915001) (width 0.25) (layer F.Cu) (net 29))
 (segment (start 68.570002 54.619998) (end 68.274999 54.915001) (width 0.25) (layer F.Cu) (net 29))
 (segment (start 65.86999 51.410012) (end 67.445001 49.835001) (width 0.25) (layer F.Cu) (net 31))
 (segment (start 65.86999 60.084992) (end 65.86999 51.410012) (width 0.25) (layer F.Cu) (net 31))
 (segment (start 66.905 61.41) (end 67.933592 61.41) (width 0.25) (layer F.Cu) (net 31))
 (segment (start 66.32 61.995) (end 66.905 61.41) (width 0.25) (layer F.Cu) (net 31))
 (segment (start 66.32 63.075002) (end 66.32 61.995) (width 0.25) (layer F.Cu) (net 31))
 (segment (start 66.905 63.660002) (end 66.32 63.075002) (width 0.25) (layer F.Cu) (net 31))
 (segment (start 68.22359 61.120002) (end 66.905 61.120002) (width 0.25) (layer F.Cu) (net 31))
 (segment (start 73.035002 58.610002) (end 67.985002 63.660002) (width 0.25) (layer F.Cu) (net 31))
 (segment (start 88.66 58.610002) (end 73.035002 58.610002) (width 0.25) (layer F.Cu) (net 31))
 (segment (start 97.070004 63.690002) (end 93.74 63.690002) (width 0.25) (layer F.Cu) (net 31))
 (segment (start 67.933592 61.41) (end 68.22359 61.120002) (width 0.25) (layer F.Cu) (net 31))
 (segment (start 97.425002 65.522004) (end 97.425002 64.045) (width 0.25) (layer F.Cu) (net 31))
 (segment (start 99.053 67.150002) (end 97.425002 65.522004) (width 0.25) (layer F.Cu) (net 31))
 (segment (start 93.74 63.690002) (end 88.66 58.610002) (width 0.25) (layer F.Cu) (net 31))
 (segment (start 108.190002 71.843) (end 103.497004 67.150002) (width 0.25) (layer F.Cu) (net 31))
 (segment (start 67.985002 63.660002) (end 66.905 63.660002) (width 0.25) (layer F.Cu) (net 31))
 (segment (start 103.497004 67.150002) (end 99.053 67.150002) (width 0.25) (layer F.Cu) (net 31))
 (segment (start 108.190002 73.025004) (end 108.190002 71.843) (width 0.25) (layer F.Cu) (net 31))
 (segment (start 66.905 61.120002) (end 65.86999 60.084992) (width 0.25) (layer F.Cu) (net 31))
 (segment (start 97.425002 64.045) (end 97.070004 63.690002) (width 0.25) (layer F.Cu) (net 31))
 (segment (start 140.719997 105.554999) (end 108.190002 73.025004) (width 0.25) (layer F.Cu) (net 31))
 (segment (start 141.510001 105.554999) (end 140.719997 105.554999) (width 0.25) (layer F.Cu) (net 31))
 (segment (start 142.009992 106.05499) (end 141.510001 105.554999) (width 0.25) (layer F.Cu) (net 31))
 (segment (start 155.171758 106.05499) (end 142.009992 106.05499) (width 0.25) (layer F.Cu) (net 31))
 (segment (start 155.45001 106.333242) (end 155.171758 106.05499) (width 0.25) (layer F.Cu) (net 31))
 (segment (start 155.45001 107.62499) (end 155.45001 106.333242) (width 0.25) (layer F.Cu) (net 31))
 (segment (start 155.125 107.95) (end 155.45001 107.62499) (width 0.25) (layer F.Cu) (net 31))
 (segment (start 154.1 107.95) (end 155.125 107.95) (width 0.25) (layer F.Cu) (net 31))
 (segment (start 97.070004 56.070002) (end 73.91 56.070002) (width 0.25) (layer F.Cu) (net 8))
 (segment (start 100.145003 59.145001) (end 97.070004 56.070002) (width 0.25) (layer F.Cu) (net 8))
 (segment (start 121.380001 59.145001) (end 100.145003 59.145001) (width 0.25) (layer F.Cu) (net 8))
 (segment (start 73.91 56.070002) (end 67.445001 62.535001) (width 0.25) (layer F.Cu) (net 8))
 (segment (start 130.710001 49.815001) (end 121.380001 59.145001) (width 0.25) (layer F.Cu) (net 8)))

